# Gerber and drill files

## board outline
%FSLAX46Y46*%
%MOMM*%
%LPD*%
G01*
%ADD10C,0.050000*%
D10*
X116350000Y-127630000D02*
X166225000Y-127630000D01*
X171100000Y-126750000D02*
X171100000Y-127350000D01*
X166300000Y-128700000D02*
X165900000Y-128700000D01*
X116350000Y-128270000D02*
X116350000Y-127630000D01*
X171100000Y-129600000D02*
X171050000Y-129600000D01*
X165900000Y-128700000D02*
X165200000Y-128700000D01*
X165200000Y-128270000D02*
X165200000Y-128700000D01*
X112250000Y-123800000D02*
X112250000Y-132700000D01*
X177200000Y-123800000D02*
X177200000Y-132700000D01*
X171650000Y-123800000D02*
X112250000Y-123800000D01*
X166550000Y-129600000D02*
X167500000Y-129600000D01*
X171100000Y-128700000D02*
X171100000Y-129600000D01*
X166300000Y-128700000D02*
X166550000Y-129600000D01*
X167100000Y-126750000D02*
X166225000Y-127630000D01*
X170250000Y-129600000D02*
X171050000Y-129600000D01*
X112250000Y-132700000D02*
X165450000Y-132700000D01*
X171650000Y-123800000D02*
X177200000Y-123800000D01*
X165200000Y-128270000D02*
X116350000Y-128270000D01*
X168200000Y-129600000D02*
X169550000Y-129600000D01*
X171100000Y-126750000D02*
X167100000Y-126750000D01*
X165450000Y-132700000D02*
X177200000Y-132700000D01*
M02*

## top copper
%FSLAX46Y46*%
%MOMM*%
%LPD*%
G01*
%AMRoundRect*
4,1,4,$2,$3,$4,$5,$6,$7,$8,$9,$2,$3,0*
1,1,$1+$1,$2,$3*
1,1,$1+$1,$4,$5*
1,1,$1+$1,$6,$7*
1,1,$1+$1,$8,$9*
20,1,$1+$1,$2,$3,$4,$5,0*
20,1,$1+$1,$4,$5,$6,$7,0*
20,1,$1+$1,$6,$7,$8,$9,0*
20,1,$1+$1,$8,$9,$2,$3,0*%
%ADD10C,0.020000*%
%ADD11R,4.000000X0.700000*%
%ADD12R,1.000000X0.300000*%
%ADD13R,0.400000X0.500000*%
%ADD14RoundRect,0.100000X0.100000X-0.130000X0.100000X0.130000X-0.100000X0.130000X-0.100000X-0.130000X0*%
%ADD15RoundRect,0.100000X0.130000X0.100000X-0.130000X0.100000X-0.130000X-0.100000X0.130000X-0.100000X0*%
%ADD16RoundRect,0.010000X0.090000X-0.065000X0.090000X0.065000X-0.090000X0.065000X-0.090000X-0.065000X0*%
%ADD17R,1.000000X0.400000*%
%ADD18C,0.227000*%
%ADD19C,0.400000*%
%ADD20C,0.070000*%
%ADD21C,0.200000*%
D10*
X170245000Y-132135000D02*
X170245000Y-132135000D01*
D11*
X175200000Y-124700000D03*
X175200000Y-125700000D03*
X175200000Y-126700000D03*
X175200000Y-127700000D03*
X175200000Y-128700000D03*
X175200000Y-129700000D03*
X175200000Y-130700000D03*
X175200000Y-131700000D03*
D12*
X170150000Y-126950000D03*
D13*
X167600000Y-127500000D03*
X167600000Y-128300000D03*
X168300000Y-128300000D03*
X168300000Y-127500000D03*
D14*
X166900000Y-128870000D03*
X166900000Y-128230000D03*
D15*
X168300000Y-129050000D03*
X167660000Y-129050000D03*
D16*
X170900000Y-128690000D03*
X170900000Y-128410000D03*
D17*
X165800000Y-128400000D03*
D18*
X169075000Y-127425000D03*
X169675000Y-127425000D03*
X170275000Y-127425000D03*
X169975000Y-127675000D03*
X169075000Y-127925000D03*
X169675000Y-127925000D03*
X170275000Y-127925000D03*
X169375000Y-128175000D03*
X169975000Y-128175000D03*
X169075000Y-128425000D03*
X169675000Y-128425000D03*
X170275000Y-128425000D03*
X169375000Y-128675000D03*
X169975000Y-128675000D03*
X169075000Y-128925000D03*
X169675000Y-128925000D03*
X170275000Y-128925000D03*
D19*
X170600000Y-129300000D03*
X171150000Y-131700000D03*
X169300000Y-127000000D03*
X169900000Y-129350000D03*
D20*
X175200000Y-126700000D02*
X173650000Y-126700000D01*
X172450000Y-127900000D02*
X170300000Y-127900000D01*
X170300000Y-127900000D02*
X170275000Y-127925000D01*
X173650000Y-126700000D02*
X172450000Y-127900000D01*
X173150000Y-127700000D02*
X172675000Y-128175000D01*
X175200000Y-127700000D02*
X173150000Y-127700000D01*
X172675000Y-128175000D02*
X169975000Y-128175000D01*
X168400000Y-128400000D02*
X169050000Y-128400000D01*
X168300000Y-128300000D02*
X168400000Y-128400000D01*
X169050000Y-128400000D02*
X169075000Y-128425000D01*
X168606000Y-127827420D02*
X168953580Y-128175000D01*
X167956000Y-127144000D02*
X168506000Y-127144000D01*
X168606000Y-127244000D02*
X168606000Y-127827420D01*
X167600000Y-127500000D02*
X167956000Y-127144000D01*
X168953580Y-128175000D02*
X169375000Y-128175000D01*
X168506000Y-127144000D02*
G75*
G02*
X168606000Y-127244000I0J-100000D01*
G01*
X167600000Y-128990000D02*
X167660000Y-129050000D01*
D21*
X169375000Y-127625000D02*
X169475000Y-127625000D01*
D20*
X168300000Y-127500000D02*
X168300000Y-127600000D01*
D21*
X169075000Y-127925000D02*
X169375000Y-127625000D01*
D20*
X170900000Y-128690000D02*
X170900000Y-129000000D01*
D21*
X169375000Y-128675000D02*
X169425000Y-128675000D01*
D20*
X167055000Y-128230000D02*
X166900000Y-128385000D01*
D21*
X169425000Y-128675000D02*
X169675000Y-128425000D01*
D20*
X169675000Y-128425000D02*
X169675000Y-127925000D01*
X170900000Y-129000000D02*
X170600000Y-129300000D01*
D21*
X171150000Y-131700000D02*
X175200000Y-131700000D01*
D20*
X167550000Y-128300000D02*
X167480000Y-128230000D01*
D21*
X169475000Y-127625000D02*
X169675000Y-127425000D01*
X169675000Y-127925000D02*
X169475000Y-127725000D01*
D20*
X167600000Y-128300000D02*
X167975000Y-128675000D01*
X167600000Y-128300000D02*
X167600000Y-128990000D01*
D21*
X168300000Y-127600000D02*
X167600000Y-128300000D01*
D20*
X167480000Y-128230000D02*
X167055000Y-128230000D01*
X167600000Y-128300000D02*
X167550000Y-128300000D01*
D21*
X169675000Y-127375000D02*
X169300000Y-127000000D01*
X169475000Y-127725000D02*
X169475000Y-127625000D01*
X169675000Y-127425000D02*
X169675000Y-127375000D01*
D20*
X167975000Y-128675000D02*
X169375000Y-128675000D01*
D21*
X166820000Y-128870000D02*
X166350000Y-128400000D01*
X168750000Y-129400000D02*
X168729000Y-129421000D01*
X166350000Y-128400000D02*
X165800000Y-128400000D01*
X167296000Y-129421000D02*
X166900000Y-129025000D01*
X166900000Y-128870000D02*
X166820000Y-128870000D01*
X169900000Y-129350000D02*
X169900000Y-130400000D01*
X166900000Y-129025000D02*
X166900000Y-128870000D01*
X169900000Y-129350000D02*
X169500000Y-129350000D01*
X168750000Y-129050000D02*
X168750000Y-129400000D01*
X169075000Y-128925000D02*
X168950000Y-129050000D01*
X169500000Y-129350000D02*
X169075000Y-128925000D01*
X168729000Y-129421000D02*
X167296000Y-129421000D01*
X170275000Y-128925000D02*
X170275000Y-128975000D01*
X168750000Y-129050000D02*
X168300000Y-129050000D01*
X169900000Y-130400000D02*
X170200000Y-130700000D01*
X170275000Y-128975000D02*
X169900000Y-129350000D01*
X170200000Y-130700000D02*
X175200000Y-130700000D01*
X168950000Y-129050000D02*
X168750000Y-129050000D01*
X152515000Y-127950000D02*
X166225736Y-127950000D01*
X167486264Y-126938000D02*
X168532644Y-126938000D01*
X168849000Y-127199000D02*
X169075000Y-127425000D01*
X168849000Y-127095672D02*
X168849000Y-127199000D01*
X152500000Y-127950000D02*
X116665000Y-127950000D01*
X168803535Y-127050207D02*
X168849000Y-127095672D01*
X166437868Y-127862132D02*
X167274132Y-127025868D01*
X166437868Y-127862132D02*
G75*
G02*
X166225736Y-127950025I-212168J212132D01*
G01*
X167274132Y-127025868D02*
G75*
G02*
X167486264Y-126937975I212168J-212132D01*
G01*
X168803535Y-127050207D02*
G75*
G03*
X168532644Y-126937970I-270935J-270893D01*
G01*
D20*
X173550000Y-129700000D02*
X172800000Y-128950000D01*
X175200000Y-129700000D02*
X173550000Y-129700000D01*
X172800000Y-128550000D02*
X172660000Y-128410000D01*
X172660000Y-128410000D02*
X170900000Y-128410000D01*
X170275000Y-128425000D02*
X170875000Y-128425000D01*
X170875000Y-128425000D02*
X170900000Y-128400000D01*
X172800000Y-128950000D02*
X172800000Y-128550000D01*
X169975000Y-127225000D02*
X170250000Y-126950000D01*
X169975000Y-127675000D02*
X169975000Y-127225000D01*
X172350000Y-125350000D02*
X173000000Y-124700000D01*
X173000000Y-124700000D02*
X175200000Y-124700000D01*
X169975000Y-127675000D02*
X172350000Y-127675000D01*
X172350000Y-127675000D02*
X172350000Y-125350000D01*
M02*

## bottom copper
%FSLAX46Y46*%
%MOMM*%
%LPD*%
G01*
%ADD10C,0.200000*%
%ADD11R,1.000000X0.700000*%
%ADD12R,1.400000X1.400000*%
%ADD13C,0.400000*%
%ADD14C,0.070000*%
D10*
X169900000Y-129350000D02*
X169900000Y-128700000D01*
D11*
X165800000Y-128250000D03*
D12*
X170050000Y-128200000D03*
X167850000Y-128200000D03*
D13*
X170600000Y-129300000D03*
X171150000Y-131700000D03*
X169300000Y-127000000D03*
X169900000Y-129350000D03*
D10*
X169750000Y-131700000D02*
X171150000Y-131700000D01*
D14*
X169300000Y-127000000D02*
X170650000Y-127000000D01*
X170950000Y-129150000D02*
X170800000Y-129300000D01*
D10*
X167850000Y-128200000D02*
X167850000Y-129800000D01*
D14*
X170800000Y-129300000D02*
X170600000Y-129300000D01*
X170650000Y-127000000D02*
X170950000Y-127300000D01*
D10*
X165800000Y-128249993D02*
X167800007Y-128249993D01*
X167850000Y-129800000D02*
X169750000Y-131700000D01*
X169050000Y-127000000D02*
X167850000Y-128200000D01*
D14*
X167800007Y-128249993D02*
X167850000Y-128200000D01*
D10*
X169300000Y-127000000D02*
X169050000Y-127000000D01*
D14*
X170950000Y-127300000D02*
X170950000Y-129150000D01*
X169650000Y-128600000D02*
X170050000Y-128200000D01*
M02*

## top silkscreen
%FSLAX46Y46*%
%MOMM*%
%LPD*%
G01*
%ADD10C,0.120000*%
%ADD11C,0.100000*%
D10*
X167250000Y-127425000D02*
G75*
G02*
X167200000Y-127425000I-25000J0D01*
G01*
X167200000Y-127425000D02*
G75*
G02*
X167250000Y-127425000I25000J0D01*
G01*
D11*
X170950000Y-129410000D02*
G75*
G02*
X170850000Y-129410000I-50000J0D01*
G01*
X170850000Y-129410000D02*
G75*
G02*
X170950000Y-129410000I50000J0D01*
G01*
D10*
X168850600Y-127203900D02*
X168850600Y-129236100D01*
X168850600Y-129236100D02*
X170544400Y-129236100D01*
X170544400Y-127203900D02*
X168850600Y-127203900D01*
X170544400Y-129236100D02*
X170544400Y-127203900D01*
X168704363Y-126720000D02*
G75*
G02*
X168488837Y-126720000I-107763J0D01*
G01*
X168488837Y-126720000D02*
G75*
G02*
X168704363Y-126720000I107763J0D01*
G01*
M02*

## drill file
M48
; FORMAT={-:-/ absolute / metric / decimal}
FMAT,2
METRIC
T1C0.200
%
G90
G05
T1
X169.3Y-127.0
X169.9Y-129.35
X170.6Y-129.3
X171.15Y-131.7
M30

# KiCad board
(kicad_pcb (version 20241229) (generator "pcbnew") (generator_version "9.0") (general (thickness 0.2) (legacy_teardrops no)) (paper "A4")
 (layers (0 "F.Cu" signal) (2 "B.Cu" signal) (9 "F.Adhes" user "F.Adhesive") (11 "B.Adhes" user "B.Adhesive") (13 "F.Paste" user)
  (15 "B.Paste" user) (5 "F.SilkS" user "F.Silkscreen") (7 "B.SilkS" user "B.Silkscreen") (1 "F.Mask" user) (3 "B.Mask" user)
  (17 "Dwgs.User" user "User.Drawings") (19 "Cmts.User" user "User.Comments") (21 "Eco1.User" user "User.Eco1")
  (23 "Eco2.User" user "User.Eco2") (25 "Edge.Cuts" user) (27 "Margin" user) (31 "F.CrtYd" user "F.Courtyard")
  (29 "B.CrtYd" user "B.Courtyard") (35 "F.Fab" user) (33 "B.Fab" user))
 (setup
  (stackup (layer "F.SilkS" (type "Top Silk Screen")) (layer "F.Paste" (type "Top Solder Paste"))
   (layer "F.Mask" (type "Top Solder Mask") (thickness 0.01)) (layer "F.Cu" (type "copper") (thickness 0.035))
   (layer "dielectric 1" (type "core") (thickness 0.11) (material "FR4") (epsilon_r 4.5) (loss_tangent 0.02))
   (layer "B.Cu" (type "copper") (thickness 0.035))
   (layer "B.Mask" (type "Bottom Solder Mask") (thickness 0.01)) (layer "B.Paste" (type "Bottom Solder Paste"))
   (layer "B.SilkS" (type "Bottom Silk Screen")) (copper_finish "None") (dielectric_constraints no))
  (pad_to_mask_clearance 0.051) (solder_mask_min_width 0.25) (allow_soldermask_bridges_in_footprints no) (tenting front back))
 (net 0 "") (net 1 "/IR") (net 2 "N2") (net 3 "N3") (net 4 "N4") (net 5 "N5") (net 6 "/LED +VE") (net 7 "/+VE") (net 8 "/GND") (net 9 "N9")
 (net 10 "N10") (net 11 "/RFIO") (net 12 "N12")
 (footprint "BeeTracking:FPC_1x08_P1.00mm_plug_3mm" (layer "F.Cu") (at 173.2 128.2)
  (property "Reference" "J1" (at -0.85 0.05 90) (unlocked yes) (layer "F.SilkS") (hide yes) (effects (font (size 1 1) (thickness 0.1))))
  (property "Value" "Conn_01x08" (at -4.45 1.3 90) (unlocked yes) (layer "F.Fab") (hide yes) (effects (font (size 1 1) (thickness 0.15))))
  (pad "1" connect rect (at 2 -3.5) (size 4 0.7) (layers "F.Cu" "F.Mask") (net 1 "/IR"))
  (pad "2" connect rect (at 2 -2.5) (size 4 0.7) (layers "F.Cu" "F.Mask") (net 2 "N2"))
  (pad "3" connect rect (at 2 -1.5) (size 4 0.7) (layers "F.Cu" "F.Mask") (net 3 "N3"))
  (pad "4" connect rect (at 2 -0.5) (size 4 0.7) (layers "F.Cu" "F.Mask") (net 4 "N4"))
  (pad "5" connect rect (at 2 0.5) (size 4 0.7) (layers "F.Cu" "F.Mask") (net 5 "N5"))
  (pad "6" connect rect (at 2 1.5) (size 4 0.7) (layers "F.Cu" "F.Mask") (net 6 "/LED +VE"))
  (pad "7" connect rect (at 2 2.5) (size 4 0.7) (layers "F.Cu" "F.Mask") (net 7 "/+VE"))
  (pad "8" connect rect (at 2 3.5) (size 4 0.7) (layers "F.Cu" "F.Mask") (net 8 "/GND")))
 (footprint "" (layer "F.Cu") (at 170.35 126.1)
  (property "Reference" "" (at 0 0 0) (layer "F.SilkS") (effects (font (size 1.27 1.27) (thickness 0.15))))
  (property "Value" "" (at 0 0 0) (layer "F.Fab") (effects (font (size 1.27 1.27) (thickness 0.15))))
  (pad "1" smd rect (at -0.2 0.85) (size 1 0.3) (layers "F.Cu" "F.Mask") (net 1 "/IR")))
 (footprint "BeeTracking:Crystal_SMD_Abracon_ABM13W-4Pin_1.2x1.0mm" (layer "F.Cu") (at 167.95 127.9 -90)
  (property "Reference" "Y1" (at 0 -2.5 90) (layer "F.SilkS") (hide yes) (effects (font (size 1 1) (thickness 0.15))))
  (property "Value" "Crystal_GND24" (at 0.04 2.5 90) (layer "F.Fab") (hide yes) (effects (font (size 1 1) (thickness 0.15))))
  (pad "1" smd rect (at -0.4 0.35 270) (size 0.5 0.4) (layers "F.Cu" "F.Mask" "F.Paste") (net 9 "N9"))
  (pad "2" smd rect (at 0.4 0.35 270) (size 0.5 0.4) (layers "F.Cu" "F.Mask" "F.Paste") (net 8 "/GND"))
  (pad "3" smd rect (at 0.4 -0.35 270) (size 0.5 0.4) (layers "F.Cu" "F.Mask" "F.Paste") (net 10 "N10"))
  (pad "4" smd rect (at -0.4 -0.35 270) (size 0.5 0.4) (layers "F.Cu" "F.Mask" "F.Paste") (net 8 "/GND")))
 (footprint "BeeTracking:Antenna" (layer "F.Cu") (at 170.245 132.135)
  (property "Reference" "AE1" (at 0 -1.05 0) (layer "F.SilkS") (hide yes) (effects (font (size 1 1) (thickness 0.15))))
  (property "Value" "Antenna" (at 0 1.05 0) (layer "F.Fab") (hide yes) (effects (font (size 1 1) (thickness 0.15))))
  (fp_line (start 0 0) (end 0 0) (stroke (width 0.02) (type solid)) (layer "F.Cu")))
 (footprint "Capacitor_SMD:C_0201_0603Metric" (layer "F.Cu") (at 166.9 128.55 90)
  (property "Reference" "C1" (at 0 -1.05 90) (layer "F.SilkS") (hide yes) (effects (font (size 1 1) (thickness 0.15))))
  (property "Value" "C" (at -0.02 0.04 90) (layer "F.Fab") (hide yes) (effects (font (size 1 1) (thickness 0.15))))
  (pad "" smd roundrect (at -0.345 0 90) (size 0.318 0.36) (layers "F.Paste") (roundrect_rratio 0.25))
  (pad "" smd roundrect (at 0.345 0 90) (size 0.318 0.36) (layers "F.Paste") (roundrect_rratio 0.25))
  (pad "1" smd roundrect (at -0.32 0 90) (size 0.46 0.4) (layers "F.Cu" "F.Mask") (roundrect_rratio 0.25) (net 7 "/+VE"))
  (pad "2" smd roundrect (at 0.32 0 90) (size 0.46 0.4) (layers "F.Cu" "F.Mask") (roundrect_rratio 0.25) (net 8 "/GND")))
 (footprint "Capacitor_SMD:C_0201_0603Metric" (layer "F.Cu") (at 167.98 129.05 180)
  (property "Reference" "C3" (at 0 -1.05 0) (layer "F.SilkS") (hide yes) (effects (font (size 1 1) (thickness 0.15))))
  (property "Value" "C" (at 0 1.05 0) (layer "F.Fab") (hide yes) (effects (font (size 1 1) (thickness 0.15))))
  (pad "" smd roundrect (at -0.345 0 180) (size 0.318 0.36) (layers "F.Paste") (roundrect_rratio 0.25))
  (pad "" smd roundrect (at 0.345 0 180) (size 0.318 0.36) (layers "F.Paste") (roundrect_rratio 0.25))
  (pad "1" smd roundrect (at -0.32 0 180) (size 0.46 0.4) (layers "F.Cu" "F.Mask") (roundrect_rratio 0.25) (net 7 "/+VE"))
  (pad "2" smd roundrect (at 0.32 0 180) (size 0.46 0.4) (layers "F.Cu" "F.Mask") (roundrect_rratio 0.25) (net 8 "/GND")))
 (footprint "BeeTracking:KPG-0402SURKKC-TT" (layer "F.Cu") (at 170.9 128.55 90)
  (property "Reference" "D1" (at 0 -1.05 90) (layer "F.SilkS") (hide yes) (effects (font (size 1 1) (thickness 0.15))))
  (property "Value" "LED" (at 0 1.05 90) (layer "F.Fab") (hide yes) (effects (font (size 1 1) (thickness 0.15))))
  (fp_circle (center -0.86 0) (end -0.81 0) (stroke (width 0.1) (type solid)) (fill no) (layer "F.SilkS"))
  (pad "" smd roundrect (at -0.14 0 90) (size 0.15 0.2) (layers "F.Mask") (roundrect_rratio 0.06666666667))
  (pad "" smd roundrect (at -0.1225 0 90) (size 0.1 0.17) (layers "F.Paste") (roundrect_rratio 0.25))
  (pad "" smd roundrect (at 0.1225 0 90) (size 0.1 0.17) (layers "F.Paste") (roundrect_rratio 0.25))
  (pad "" smd roundrect (at 0.14 0 90) (size 0.15 0.2) (layers "F.Mask") (roundrect_rratio 0.06666666667))
  (pad "1" smd roundrect (at -0.14 0 90) (size 0.15 0.2) (layers "F.Cu" "F.Mask") (roundrect_rratio 0.06666666667) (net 8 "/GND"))
  (pad "2" smd roundrect (at 0.14 0 90) (size 0.15 0.2) (layers "F.Cu" "F.Mask") (roundrect_rratio 0.06666666667) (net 6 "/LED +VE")))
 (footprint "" (layer "F.Cu") (at 166 127.6)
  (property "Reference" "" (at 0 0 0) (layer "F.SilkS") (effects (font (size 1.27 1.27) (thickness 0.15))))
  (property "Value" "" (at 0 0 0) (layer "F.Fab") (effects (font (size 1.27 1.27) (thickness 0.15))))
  (pad "1" smd rect (at -0.2 0.8) (size 1 0.4) (layers "F.Cu" "F.Mask") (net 7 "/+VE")))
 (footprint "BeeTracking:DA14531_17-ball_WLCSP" (layer "F.Cu") (at 169.697 128.22)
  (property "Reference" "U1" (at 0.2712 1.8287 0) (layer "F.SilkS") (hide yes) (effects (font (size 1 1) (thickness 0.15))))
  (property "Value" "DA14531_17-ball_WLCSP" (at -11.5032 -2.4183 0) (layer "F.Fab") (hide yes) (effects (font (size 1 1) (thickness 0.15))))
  (fp_line (start -0.8464 -1.0161) (end -0.8464 1.0161) (stroke (width 0.12) (type solid)) (layer "F.SilkS"))
  (fp_line (start -0.8464 1.0161) (end 0.8474 1.0161) (stroke (width 0.12) (type solid)) (layer "F.SilkS"))
  (fp_line (start 0.8474 -1.0161) (end -0.8464 -1.0161) (stroke (width 0.12) (type solid)) (layer "F.SilkS"))
  (fp_line (start 0.8474 1.0161) (end 0.8474 -1.0161) (stroke (width 0.12) (type solid)) (layer "F.SilkS"))
  (fp_circle (center -1.1004 -1.5) (end -1.0242 -1.4238) (stroke (width 0.12) (type solid)) (fill no) (layer "F.SilkS"))
  (pad "A1" smd circle (at -0.622 -0.795) (size 0.227 0.227) (layers "F.Cu" "F.Mask" "F.Paste") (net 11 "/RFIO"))
  (pad "A3" smd circle (at -0.022 -0.795) (size 0.227 0.227) (layers "F.Cu" "F.Mask" "F.Paste") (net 8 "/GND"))
  (pad "A5" smd circle (at 0.578 -0.795) (size 0.227 0.227) (layers "F.Cu" "F.Mask" "F.Paste") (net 2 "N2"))
  (pad "B4" smd circle (at 0.278 -0.545) (size 0.227 0.227) (layers "F.Cu" "F.Mask" "F.Paste") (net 1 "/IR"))
  (pad "C1" smd circle (at -0.622 -0.295) (size 0.227 0.227) (layers "F.Cu" "F.Mask" "F.Paste") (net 8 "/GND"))
  (pad "C3" smd circle (at -0.022 -0.295) (size 0.227 0.227) (layers "F.Cu" "F.Mask" "F.Paste") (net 8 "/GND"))
  (pad "C5" smd circle (at 0.578 -0.295) (size 0.227 0.227) (layers "F.Cu" "F.Mask" "F.Paste") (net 3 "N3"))
  (pad "D2" smd circle (at -0.322 -0.045) (size 0.227 0.227) (layers "F.Cu" "F.Mask" "F.Paste") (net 9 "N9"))
  (pad "D4" smd circle (at 0.278 -0.045) (size 0.227 0.227) (layers "F.Cu" "F.Mask" "F.Paste") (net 4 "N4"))
  (pad "E1" smd circle (at -0.622 0.205) (size 0.227 0.227) (layers "F.Cu" "F.Mask" "F.Paste") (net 10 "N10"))
  (pad "E3" smd circle (at -0.022 0.205) (size 0.227 0.227) (layers "F.Cu" "F.Mask" "F.Paste") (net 8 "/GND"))
  (pad "E5" smd circle (at 0.578 0.205) (size 0.227 0.227) (layers "F.Cu" "F.Mask" "F.Paste") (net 6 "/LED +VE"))
  (pad "F2" smd circle (at -0.322 0.455) (size 0.227 0.227) (layers "F.Cu" "F.Mask" "F.Paste") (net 8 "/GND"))
  (pad "F4" smd circle (at 0.278 0.455) (size 0.227 0.227) (layers "F.Cu" "F.Mask" "F.Paste") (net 5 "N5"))
  (pad "G1" smd circle (at -0.622 0.705) (size 0.227 0.227) (layers "F.Cu" "F.Mask" "F.Paste") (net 7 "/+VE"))
  (pad "G3" smd circle (at -0.022 0.705) (size 0.227 0.227) (layers "F.Cu" "F.Mask" "F.Paste") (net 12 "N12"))
  (pad "G5" smd circle (at 0.578 0.705) (size 0.227 0.227) (layers "F.Cu" "F.Mask" "F.Paste") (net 7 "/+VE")))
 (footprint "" (layer "B.Cu") (at 165.8 128.4 180)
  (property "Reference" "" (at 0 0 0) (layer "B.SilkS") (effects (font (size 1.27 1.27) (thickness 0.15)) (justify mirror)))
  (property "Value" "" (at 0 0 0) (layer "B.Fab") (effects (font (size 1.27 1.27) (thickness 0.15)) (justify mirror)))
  (pad "1" smd rect (at 0 0.15 180) (size 1 0.7) (layers "B.Cu" "B.Mask") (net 8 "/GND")))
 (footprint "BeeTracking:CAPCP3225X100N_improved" (layer "B.Cu") (at 168.95 128.2 180)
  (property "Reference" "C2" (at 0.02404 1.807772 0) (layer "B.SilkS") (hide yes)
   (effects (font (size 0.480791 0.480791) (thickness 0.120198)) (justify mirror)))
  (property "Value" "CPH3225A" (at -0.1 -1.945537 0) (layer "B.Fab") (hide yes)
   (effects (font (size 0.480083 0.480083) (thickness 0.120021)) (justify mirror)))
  (pad "1" smd rect (at -1.1 0) (size 1.4 1.4) (layers "B.Cu" "B.Mask" "B.Paste") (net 7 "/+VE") (solder_mask_margin 0.102))
  (pad "2" smd rect (at 1.1 0) (size 1.4 1.4) (layers "B.Cu" "B.Mask" "B.Paste") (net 8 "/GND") (solder_mask_margin 0.102)))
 (gr_line (start 169.9 129.35) (end 169.9 128.7) (stroke (width 0.2) (type default)) (layer "B.Cu") (net 7))
 (gr_circle (center 167.225 127.425) (end 167.25 127.425) (stroke (width 0.12) (type default)) (fill no) (layer "F.SilkS"))
 (gr_line (start 116.35 127.63) (end 166.225 127.63) (stroke (width 0.05) (type default)) (layer "Edge.Cuts"))
 (gr_line (start 171.1 126.75) (end 171.1 127.35) (stroke (width 0.05) (type default)) (layer "Edge.Cuts"))
 (gr_line (start 166.3 128.7) (end 165.9 128.7) (stroke (width 0.05) (type default)) (layer "Edge.Cuts"))
 (gr_line (start 116.35 128.27) (end 116.35 127.63) (stroke (width 0.05) (type default)) (layer "Edge.Cuts"))
 (gr_line (start 171.1 129.6) (end 171.05 129.6) (stroke (width 0.05) (type default)) (layer "Edge.Cuts"))
 (gr_line (start 165.9 128.7) (end 165.2 128.7) (stroke (width 0.05) (type default)) (layer "Edge.Cuts"))
 (gr_line (start 165.2 128.27) (end 165.2 128.7) (stroke (width 0.05) (type default)) (layer "Edge.Cuts"))
 (gr_line (start 112.25 123.8) (end 112.25 132.7) (stroke (width 0.05) (type default)) (layer "Edge.Cuts"))
 (gr_line (start 177.2 123.8) (end 177.2 132.7) (stroke (width 0.05) (type default)) (layer "Edge.Cuts"))
 (gr_line (start 171.65 123.8) (end 112.25 123.8) (stroke (width 0.05) (type default)) (layer "Edge.Cuts"))
 (gr_line (start 166.55 129.6) (end 167.5 129.6) (stroke (width 0.05) (type default)) (layer "Edge.Cuts"))
 (gr_line (start 171.1 128.7) (end 171.1 129.6) (stroke (width 0.05) (type default)) (layer "Edge.Cuts"))
 (gr_line (start 166.3 128.7) (end 166.55 129.6) (stroke (width 0.05) (type default)) (layer "Edge.Cuts"))
 (gr_line (start 167.1 126.75) (end 166.225 127.63) (stroke (width 0.05) (type default)) (layer "Edge.Cuts"))
 (gr_line (start 170.25 129.6) (end 171.05 129.6) (stroke (width 0.05) (type default)) (layer "Edge.Cuts"))
 (gr_line (start 112.25 132.7) (end 165.45 132.7) (stroke (width 0.05) (type default)) (layer "Edge.Cuts"))
 (gr_line (start 171.65 123.8) (end 177.2 123.8) (stroke (width 0.05) (type default)) (layer "Edge.Cuts"))
 (gr_line (start 165.2 128.27) (end 116.35 128.27) (stroke (width 0.05) (type default)) (layer "Edge.Cuts"))
 (gr_line (start 168.2 129.6) (end 169.55 129.6) (stroke (width 0.05) (type default)) (layer "Edge.Cuts"))
 (gr_line (start 171.1 126.75) (end 167.1 126.75) (stroke (width 0.05) (type default)) (layer "Edge.Cuts"))
 (gr_line (start 165.45 132.7) (end 177.2 132.7) (stroke (width 0.05) (type default)) (layer "Edge.Cuts"))
 (segment (start 175.2 126.7) (end 173.65 126.7) (width 0.07) (layer "F.Cu") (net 3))
 (segment (start 172.45 127.9) (end 170.3 127.9) (width 0.07) (layer "F.Cu") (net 3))
 (segment (start 170.3 127.9) (end 170.275 127.925) (width 0.07) (layer "F.Cu") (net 3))
 (segment (start 173.65 126.7) (end 172.45 127.9) (width 0.07) (layer "F.Cu") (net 3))
 (segment (start 173.15 127.7) (end 172.675 128.175) (width 0.07) (layer "F.Cu") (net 4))
 (segment (start 175.2 127.7) (end 173.15 127.7) (width 0.07) (layer "F.Cu") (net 4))
 (segment (start 172.675 128.175) (end 169.975 128.175) (width 0.07) (layer "F.Cu") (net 4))
 (segment (start 168.4 128.4) (end 169.05 128.4) (width 0.07) (layer "F.Cu") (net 10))
 (segment (start 168.3 128.3) (end 168.4 128.4) (width 0.07) (layer "F.Cu") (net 10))
 (segment (start 169.05 128.4) (end 169.075 128.425) (width 0.07) (layer "F.Cu") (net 10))
 (segment (start 168.606 127.82742) (end 168.95358 128.175) (width 0.07) (layer "F.Cu") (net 9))
 (segment (start 167.956 127.144) (end 168.506 127.144) (width 0.07) (layer "F.Cu") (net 9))
 (segment (start 168.606 127.244) (end 168.606 127.82742) (width 0.07) (layer "F.Cu") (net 9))
 (segment (start 167.6 127.5) (end 167.956 127.144) (width 0.07) (layer "F.Cu") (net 9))
 (segment (start 168.95358 128.175) (end 169.375 128.175) (width 0.07) (layer "F.Cu") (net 9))
 (arc (start 168.506 127.144) (mid 168.576711 127.173289) (end 168.606 127.244) (width 0.07) (layer "F.Cu") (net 9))
 (segment (start 167.6 128.99) (end 167.66 129.05) (width 0.07) (layer "F.Cu") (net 8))
 (segment (start 169.375 127.625) (end 169.475 127.625) (width 0.2) (layer "F.Cu") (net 8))
 (segment (start 168.3 127.5) (end 168.3 127.6) (width 0.07) (layer "F.Cu") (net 8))
 (segment (start 169.075 127.925) (end 169.375 127.625) (width 0.2) (layer "F.Cu") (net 8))
 (segment (start 170.9 128.69) (end 170.9 129) (width 0.07) (layer "F.Cu") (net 8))
 (segment (start 169.375 128.675) (end 169.425 128.675) (width 0.2) (layer "F.Cu") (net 8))
 (segment (start 167.055 128.23) (end 166.9 128.385) (width 0.07) (layer "F.Cu") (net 8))
 (segment (start 169.425 128.675) (end 169.675 128.425) (width 0.2) (layer "F.Cu") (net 8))
 (segment (start 169.675 128.425) (end 169.675 127.925) (width 0.07) (layer "F.Cu") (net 8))
 (segment (start 170.9 129) (end 170.6 129.3) (width 0.07) (layer "F.Cu") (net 8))
 (segment (start 171.15 131.7) (end 175.2 131.7) (width 0.2) (layer "F.Cu") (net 8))
 (segment (start 167.55 128.3) (end 167.48 128.23) (width 0.07) (layer "F.Cu") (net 8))
 (segment (start 169.475 127.625) (end 169.675 127.425) (width 0.2) (layer "F.Cu") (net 8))
 (segment (start 169.675 127.925) (end 169.475 127.725) (width 0.2) (layer "F.Cu") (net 8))
 (segment (start 167.6 128.3) (end 167.975 128.675) (width 0.07) (layer "F.Cu") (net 8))
 (segment (start 167.6 128.3) (end 167.6 128.99) (width 0.07) (layer "F.Cu") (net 8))
 (segment (start 168.3 127.6) (end 167.6 128.3) (width 0.2) (layer "F.Cu") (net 8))
 (segment (start 167.48 128.23) (end 167.055 128.23) (width 0.07) (layer "F.Cu") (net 8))
 (segment (start 167.6 128.3) (end 167.55 128.3) (width 0.07) (layer "F.Cu") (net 8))
 (segment (start 169.675 127.375) (end 169.3 127) (width 0.2) (layer "F.Cu") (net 8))
 (segment (start 169.475 127.725) (end 169.475 127.625) (width 0.2) (layer "F.Cu") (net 8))
 (segment (start 169.675 127.425) (end 169.675 127.375) (width 0.2) (layer "F.Cu") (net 8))
 (segment (start 167.975 128.675) (end 169.375 128.675) (width 0.07) (layer "F.Cu") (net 8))
 (via (at 170.6 129.3) (size 0.4) (drill 0.2) (layers "F.Cu" "B.Cu") (free yes) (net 8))
 (via (at 171.15 131.7) (size 0.4) (drill 0.2) (layers "F.Cu" "B.Cu") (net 8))
 (via (at 169.3 127) (size 0.4) (drill 0.2) (layers "F.Cu" "B.Cu") (free yes) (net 8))
 (segment (start 169.75 131.7) (end 171.15 131.7) (width 0.2) (layer "B.Cu") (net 8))
 (segment (start 169.3 127) (end 170.65 127) (width 0.07) (layer "B.Cu") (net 8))
 (segment (start 170.95 129.15) (end 170.8 129.3) (width 0.07) (layer "B.Cu") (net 8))
 (segment (start 167.85 128.2) (end 167.85 129.8) (width 0.2) (layer "B.Cu") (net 8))
 (segment (start 170.8 129.3) (end 170.6 129.3) (width 0.07) (layer "B.Cu") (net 8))
 (segment (start 170.65 127) (end 170.95 127.3) (width 0.07) (layer "B.Cu") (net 8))
 (segment (start 165.8 128.249993) (end 167.800007 128.249993) (width 0.2) (layer "B.Cu") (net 8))
 (segment (start 167.85 129.8) (end 169.75 131.7) (width 0.2) (layer "B.Cu") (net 8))
 (segment (start 169.05 127) (end 167.85 128.2) (width 0.2) (layer "B.Cu") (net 8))
 (segment (start 167.800007 128.249993) (end 167.85 128.2) (width 0.07) (layer "B.Cu") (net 8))
 (segment (start 169.3 127) (end 169.05 127) (width 0.2) (layer "B.Cu") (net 8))
 (segment (start 170.95 127.3) (end 170.95 129.15) (width 0.07) (layer "B.Cu") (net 8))
 (segment (start 166.82 128.87) (end 166.35 128.4) (width 0.2) (layer "F.Cu") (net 7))
 (segment (start 168.75 129.4) (end 168.729 129.421) (width 0.2) (layer "F.Cu") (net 7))
 (segment (start 166.35 128.4) (end 165.8 128.4) (width 0.2) (layer "F.Cu") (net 7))
 (segment (start 167.296 129.421) (end 166.9 129.025) (width 0.2) (layer "F.Cu") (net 7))
 (segment (start 166.9 128.87) (end 166.82 128.87) (width 0.2) (layer "F.Cu") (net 7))
 (segment (start 169.9 129.35) (end 169.9 130.4) (width 0.2) (layer "F.Cu") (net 7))
 (segment (start 166.9 129.025) (end 166.9 128.87) (width 0.2) (layer "F.Cu") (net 7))
 (segment (start 169.9 129.35) (end 169.5 129.35) (width 0.2) (layer "F.Cu") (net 7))
 (segment (start 168.75 129.05) (end 168.75 129.4) (width 0.2) (layer "F.Cu") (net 7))
 (segment (start 169.075 128.925) (end 168.95 129.05) (width 0.2) (layer "F.Cu") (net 7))
 (segment (start 169.5 129.35) (end 169.075 128.925) (width 0.2) (layer "F.Cu") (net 7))
 (segment (start 168.729 129.421) (end 167.296 129.421) (width 0.2) (layer "F.Cu") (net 7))
 (segment (start 170.275 128.925) (end 170.275 128.975) (width 0.2) (layer "F.Cu") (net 7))
 (segment (start 168.75 129.05) (end 168.3 129.05) (width 0.2) (layer "F.Cu") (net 7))
 (segment (start 169.9 130.4) (end 170.2 130.7) (width 0.2) (layer "F.Cu") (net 7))
 (segment (start 170.275 128.975) (end 169.9 129.35) (width 0.2) (layer "F.Cu") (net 7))
 (segment (start 170.2 130.7) (end 175.2 130.7) (width 0.2) (layer "F.Cu") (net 7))
 (segment (start 168.95 129.05) (end 168.75 129.05) (width 0.2) (layer "F.Cu") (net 7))
 (via (at 169.9 129.35) (size 0.4) (drill 0.2) (layers "F.Cu" "B.Cu") (free yes) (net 7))
 (segment (start 169.65 128.6) (end 170.05 128.2) (width 0.07) (layer "B.Cu") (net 7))
 (segment (start 152.515 127.95) (end 166.225736 127.95) (width 0.2) (layer "F.Cu") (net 11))
 (segment (start 167.486264 126.938) (end 168.532644 126.938) (width 0.2) (layer "F.Cu") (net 11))
 (segment (start 168.849 127.199) (end 169.075 127.425) (width 0.2) (layer "F.Cu") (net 11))
 (segment (start 168.849 127.095672) (end 168.849 127.199) (width 0.2) (layer "F.Cu") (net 11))
 (segment (start 152.5 127.95) (end 116.665 127.95) (width 0.2) (layer "F.Cu") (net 11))
 (segment (start 168.803535 127.050207) (end 168.849 127.095672) (width 0.2) (layer "F.Cu") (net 11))
 (segment (start 166.437868 127.862132) (end 167.274132 127.025868) (width 0.2) (layer "F.Cu") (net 11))
 (arc (start 166.437868 127.862132) (mid 166.340541 127.927164) (end 166.225736 127.95) (width 0.2) (layer "F.Cu") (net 11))
 (arc (start 167.274132 127.025868) (mid 167.371459 126.960836) (end 167.486264 126.938) (width 0.2) (layer "F.Cu") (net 11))
 (arc (start 168.803535 127.050207) (mid 168.679249 126.967162) (end 168.532644 126.938) (width 0.2) (layer "F.Cu") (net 11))
 (segment (start 173.55 129.7) (end 172.8 128.95) (width 0.07) (layer "F.Cu") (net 6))
 (segment (start 175.2 129.7) (end 173.55 129.7) (width 0.07) (layer "F.Cu") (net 6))
 (segment (start 172.8 128.55) (end 172.66 128.41) (width 0.07) (layer "F.Cu") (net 6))
 (segment (start 172.66 128.41) (end 170.9 128.41) (width 0.07) (layer "F.Cu") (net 6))
 (segment (start 170.275 128.425) (end 170.875 128.425) (width 0.07) (layer "F.Cu") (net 6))
 (segment (start 170.875 128.425) (end 170.9 128.4) (width 0.07) (layer "F.Cu") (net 6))
 (segment (start 172.8 128.95) (end 172.8 128.55) (width 0.07) (layer "F.Cu") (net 6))
 (segment (start 169.975 127.225) (end 170.25 126.95) (width 0.07) (layer "F.Cu") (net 1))
 (segment (start 169.975 127.675) (end 169.975 127.225) (width 0.07) (layer "F.Cu") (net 1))
 (segment (start 172.35 125.35) (end 173 124.7) (width 0.07) (layer "F.Cu") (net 1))
 (segment (start 173 124.7) (end 175.2 124.7) (width 0.07) (layer "F.Cu") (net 1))
 (segment (start 169.975 127.675) (end 172.35 127.675) (width 0.07) (layer "F.Cu") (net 1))
 (segment (start 172.35 127.675) (end 172.35 125.35) (width 0.07) (layer "F.Cu") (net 1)))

